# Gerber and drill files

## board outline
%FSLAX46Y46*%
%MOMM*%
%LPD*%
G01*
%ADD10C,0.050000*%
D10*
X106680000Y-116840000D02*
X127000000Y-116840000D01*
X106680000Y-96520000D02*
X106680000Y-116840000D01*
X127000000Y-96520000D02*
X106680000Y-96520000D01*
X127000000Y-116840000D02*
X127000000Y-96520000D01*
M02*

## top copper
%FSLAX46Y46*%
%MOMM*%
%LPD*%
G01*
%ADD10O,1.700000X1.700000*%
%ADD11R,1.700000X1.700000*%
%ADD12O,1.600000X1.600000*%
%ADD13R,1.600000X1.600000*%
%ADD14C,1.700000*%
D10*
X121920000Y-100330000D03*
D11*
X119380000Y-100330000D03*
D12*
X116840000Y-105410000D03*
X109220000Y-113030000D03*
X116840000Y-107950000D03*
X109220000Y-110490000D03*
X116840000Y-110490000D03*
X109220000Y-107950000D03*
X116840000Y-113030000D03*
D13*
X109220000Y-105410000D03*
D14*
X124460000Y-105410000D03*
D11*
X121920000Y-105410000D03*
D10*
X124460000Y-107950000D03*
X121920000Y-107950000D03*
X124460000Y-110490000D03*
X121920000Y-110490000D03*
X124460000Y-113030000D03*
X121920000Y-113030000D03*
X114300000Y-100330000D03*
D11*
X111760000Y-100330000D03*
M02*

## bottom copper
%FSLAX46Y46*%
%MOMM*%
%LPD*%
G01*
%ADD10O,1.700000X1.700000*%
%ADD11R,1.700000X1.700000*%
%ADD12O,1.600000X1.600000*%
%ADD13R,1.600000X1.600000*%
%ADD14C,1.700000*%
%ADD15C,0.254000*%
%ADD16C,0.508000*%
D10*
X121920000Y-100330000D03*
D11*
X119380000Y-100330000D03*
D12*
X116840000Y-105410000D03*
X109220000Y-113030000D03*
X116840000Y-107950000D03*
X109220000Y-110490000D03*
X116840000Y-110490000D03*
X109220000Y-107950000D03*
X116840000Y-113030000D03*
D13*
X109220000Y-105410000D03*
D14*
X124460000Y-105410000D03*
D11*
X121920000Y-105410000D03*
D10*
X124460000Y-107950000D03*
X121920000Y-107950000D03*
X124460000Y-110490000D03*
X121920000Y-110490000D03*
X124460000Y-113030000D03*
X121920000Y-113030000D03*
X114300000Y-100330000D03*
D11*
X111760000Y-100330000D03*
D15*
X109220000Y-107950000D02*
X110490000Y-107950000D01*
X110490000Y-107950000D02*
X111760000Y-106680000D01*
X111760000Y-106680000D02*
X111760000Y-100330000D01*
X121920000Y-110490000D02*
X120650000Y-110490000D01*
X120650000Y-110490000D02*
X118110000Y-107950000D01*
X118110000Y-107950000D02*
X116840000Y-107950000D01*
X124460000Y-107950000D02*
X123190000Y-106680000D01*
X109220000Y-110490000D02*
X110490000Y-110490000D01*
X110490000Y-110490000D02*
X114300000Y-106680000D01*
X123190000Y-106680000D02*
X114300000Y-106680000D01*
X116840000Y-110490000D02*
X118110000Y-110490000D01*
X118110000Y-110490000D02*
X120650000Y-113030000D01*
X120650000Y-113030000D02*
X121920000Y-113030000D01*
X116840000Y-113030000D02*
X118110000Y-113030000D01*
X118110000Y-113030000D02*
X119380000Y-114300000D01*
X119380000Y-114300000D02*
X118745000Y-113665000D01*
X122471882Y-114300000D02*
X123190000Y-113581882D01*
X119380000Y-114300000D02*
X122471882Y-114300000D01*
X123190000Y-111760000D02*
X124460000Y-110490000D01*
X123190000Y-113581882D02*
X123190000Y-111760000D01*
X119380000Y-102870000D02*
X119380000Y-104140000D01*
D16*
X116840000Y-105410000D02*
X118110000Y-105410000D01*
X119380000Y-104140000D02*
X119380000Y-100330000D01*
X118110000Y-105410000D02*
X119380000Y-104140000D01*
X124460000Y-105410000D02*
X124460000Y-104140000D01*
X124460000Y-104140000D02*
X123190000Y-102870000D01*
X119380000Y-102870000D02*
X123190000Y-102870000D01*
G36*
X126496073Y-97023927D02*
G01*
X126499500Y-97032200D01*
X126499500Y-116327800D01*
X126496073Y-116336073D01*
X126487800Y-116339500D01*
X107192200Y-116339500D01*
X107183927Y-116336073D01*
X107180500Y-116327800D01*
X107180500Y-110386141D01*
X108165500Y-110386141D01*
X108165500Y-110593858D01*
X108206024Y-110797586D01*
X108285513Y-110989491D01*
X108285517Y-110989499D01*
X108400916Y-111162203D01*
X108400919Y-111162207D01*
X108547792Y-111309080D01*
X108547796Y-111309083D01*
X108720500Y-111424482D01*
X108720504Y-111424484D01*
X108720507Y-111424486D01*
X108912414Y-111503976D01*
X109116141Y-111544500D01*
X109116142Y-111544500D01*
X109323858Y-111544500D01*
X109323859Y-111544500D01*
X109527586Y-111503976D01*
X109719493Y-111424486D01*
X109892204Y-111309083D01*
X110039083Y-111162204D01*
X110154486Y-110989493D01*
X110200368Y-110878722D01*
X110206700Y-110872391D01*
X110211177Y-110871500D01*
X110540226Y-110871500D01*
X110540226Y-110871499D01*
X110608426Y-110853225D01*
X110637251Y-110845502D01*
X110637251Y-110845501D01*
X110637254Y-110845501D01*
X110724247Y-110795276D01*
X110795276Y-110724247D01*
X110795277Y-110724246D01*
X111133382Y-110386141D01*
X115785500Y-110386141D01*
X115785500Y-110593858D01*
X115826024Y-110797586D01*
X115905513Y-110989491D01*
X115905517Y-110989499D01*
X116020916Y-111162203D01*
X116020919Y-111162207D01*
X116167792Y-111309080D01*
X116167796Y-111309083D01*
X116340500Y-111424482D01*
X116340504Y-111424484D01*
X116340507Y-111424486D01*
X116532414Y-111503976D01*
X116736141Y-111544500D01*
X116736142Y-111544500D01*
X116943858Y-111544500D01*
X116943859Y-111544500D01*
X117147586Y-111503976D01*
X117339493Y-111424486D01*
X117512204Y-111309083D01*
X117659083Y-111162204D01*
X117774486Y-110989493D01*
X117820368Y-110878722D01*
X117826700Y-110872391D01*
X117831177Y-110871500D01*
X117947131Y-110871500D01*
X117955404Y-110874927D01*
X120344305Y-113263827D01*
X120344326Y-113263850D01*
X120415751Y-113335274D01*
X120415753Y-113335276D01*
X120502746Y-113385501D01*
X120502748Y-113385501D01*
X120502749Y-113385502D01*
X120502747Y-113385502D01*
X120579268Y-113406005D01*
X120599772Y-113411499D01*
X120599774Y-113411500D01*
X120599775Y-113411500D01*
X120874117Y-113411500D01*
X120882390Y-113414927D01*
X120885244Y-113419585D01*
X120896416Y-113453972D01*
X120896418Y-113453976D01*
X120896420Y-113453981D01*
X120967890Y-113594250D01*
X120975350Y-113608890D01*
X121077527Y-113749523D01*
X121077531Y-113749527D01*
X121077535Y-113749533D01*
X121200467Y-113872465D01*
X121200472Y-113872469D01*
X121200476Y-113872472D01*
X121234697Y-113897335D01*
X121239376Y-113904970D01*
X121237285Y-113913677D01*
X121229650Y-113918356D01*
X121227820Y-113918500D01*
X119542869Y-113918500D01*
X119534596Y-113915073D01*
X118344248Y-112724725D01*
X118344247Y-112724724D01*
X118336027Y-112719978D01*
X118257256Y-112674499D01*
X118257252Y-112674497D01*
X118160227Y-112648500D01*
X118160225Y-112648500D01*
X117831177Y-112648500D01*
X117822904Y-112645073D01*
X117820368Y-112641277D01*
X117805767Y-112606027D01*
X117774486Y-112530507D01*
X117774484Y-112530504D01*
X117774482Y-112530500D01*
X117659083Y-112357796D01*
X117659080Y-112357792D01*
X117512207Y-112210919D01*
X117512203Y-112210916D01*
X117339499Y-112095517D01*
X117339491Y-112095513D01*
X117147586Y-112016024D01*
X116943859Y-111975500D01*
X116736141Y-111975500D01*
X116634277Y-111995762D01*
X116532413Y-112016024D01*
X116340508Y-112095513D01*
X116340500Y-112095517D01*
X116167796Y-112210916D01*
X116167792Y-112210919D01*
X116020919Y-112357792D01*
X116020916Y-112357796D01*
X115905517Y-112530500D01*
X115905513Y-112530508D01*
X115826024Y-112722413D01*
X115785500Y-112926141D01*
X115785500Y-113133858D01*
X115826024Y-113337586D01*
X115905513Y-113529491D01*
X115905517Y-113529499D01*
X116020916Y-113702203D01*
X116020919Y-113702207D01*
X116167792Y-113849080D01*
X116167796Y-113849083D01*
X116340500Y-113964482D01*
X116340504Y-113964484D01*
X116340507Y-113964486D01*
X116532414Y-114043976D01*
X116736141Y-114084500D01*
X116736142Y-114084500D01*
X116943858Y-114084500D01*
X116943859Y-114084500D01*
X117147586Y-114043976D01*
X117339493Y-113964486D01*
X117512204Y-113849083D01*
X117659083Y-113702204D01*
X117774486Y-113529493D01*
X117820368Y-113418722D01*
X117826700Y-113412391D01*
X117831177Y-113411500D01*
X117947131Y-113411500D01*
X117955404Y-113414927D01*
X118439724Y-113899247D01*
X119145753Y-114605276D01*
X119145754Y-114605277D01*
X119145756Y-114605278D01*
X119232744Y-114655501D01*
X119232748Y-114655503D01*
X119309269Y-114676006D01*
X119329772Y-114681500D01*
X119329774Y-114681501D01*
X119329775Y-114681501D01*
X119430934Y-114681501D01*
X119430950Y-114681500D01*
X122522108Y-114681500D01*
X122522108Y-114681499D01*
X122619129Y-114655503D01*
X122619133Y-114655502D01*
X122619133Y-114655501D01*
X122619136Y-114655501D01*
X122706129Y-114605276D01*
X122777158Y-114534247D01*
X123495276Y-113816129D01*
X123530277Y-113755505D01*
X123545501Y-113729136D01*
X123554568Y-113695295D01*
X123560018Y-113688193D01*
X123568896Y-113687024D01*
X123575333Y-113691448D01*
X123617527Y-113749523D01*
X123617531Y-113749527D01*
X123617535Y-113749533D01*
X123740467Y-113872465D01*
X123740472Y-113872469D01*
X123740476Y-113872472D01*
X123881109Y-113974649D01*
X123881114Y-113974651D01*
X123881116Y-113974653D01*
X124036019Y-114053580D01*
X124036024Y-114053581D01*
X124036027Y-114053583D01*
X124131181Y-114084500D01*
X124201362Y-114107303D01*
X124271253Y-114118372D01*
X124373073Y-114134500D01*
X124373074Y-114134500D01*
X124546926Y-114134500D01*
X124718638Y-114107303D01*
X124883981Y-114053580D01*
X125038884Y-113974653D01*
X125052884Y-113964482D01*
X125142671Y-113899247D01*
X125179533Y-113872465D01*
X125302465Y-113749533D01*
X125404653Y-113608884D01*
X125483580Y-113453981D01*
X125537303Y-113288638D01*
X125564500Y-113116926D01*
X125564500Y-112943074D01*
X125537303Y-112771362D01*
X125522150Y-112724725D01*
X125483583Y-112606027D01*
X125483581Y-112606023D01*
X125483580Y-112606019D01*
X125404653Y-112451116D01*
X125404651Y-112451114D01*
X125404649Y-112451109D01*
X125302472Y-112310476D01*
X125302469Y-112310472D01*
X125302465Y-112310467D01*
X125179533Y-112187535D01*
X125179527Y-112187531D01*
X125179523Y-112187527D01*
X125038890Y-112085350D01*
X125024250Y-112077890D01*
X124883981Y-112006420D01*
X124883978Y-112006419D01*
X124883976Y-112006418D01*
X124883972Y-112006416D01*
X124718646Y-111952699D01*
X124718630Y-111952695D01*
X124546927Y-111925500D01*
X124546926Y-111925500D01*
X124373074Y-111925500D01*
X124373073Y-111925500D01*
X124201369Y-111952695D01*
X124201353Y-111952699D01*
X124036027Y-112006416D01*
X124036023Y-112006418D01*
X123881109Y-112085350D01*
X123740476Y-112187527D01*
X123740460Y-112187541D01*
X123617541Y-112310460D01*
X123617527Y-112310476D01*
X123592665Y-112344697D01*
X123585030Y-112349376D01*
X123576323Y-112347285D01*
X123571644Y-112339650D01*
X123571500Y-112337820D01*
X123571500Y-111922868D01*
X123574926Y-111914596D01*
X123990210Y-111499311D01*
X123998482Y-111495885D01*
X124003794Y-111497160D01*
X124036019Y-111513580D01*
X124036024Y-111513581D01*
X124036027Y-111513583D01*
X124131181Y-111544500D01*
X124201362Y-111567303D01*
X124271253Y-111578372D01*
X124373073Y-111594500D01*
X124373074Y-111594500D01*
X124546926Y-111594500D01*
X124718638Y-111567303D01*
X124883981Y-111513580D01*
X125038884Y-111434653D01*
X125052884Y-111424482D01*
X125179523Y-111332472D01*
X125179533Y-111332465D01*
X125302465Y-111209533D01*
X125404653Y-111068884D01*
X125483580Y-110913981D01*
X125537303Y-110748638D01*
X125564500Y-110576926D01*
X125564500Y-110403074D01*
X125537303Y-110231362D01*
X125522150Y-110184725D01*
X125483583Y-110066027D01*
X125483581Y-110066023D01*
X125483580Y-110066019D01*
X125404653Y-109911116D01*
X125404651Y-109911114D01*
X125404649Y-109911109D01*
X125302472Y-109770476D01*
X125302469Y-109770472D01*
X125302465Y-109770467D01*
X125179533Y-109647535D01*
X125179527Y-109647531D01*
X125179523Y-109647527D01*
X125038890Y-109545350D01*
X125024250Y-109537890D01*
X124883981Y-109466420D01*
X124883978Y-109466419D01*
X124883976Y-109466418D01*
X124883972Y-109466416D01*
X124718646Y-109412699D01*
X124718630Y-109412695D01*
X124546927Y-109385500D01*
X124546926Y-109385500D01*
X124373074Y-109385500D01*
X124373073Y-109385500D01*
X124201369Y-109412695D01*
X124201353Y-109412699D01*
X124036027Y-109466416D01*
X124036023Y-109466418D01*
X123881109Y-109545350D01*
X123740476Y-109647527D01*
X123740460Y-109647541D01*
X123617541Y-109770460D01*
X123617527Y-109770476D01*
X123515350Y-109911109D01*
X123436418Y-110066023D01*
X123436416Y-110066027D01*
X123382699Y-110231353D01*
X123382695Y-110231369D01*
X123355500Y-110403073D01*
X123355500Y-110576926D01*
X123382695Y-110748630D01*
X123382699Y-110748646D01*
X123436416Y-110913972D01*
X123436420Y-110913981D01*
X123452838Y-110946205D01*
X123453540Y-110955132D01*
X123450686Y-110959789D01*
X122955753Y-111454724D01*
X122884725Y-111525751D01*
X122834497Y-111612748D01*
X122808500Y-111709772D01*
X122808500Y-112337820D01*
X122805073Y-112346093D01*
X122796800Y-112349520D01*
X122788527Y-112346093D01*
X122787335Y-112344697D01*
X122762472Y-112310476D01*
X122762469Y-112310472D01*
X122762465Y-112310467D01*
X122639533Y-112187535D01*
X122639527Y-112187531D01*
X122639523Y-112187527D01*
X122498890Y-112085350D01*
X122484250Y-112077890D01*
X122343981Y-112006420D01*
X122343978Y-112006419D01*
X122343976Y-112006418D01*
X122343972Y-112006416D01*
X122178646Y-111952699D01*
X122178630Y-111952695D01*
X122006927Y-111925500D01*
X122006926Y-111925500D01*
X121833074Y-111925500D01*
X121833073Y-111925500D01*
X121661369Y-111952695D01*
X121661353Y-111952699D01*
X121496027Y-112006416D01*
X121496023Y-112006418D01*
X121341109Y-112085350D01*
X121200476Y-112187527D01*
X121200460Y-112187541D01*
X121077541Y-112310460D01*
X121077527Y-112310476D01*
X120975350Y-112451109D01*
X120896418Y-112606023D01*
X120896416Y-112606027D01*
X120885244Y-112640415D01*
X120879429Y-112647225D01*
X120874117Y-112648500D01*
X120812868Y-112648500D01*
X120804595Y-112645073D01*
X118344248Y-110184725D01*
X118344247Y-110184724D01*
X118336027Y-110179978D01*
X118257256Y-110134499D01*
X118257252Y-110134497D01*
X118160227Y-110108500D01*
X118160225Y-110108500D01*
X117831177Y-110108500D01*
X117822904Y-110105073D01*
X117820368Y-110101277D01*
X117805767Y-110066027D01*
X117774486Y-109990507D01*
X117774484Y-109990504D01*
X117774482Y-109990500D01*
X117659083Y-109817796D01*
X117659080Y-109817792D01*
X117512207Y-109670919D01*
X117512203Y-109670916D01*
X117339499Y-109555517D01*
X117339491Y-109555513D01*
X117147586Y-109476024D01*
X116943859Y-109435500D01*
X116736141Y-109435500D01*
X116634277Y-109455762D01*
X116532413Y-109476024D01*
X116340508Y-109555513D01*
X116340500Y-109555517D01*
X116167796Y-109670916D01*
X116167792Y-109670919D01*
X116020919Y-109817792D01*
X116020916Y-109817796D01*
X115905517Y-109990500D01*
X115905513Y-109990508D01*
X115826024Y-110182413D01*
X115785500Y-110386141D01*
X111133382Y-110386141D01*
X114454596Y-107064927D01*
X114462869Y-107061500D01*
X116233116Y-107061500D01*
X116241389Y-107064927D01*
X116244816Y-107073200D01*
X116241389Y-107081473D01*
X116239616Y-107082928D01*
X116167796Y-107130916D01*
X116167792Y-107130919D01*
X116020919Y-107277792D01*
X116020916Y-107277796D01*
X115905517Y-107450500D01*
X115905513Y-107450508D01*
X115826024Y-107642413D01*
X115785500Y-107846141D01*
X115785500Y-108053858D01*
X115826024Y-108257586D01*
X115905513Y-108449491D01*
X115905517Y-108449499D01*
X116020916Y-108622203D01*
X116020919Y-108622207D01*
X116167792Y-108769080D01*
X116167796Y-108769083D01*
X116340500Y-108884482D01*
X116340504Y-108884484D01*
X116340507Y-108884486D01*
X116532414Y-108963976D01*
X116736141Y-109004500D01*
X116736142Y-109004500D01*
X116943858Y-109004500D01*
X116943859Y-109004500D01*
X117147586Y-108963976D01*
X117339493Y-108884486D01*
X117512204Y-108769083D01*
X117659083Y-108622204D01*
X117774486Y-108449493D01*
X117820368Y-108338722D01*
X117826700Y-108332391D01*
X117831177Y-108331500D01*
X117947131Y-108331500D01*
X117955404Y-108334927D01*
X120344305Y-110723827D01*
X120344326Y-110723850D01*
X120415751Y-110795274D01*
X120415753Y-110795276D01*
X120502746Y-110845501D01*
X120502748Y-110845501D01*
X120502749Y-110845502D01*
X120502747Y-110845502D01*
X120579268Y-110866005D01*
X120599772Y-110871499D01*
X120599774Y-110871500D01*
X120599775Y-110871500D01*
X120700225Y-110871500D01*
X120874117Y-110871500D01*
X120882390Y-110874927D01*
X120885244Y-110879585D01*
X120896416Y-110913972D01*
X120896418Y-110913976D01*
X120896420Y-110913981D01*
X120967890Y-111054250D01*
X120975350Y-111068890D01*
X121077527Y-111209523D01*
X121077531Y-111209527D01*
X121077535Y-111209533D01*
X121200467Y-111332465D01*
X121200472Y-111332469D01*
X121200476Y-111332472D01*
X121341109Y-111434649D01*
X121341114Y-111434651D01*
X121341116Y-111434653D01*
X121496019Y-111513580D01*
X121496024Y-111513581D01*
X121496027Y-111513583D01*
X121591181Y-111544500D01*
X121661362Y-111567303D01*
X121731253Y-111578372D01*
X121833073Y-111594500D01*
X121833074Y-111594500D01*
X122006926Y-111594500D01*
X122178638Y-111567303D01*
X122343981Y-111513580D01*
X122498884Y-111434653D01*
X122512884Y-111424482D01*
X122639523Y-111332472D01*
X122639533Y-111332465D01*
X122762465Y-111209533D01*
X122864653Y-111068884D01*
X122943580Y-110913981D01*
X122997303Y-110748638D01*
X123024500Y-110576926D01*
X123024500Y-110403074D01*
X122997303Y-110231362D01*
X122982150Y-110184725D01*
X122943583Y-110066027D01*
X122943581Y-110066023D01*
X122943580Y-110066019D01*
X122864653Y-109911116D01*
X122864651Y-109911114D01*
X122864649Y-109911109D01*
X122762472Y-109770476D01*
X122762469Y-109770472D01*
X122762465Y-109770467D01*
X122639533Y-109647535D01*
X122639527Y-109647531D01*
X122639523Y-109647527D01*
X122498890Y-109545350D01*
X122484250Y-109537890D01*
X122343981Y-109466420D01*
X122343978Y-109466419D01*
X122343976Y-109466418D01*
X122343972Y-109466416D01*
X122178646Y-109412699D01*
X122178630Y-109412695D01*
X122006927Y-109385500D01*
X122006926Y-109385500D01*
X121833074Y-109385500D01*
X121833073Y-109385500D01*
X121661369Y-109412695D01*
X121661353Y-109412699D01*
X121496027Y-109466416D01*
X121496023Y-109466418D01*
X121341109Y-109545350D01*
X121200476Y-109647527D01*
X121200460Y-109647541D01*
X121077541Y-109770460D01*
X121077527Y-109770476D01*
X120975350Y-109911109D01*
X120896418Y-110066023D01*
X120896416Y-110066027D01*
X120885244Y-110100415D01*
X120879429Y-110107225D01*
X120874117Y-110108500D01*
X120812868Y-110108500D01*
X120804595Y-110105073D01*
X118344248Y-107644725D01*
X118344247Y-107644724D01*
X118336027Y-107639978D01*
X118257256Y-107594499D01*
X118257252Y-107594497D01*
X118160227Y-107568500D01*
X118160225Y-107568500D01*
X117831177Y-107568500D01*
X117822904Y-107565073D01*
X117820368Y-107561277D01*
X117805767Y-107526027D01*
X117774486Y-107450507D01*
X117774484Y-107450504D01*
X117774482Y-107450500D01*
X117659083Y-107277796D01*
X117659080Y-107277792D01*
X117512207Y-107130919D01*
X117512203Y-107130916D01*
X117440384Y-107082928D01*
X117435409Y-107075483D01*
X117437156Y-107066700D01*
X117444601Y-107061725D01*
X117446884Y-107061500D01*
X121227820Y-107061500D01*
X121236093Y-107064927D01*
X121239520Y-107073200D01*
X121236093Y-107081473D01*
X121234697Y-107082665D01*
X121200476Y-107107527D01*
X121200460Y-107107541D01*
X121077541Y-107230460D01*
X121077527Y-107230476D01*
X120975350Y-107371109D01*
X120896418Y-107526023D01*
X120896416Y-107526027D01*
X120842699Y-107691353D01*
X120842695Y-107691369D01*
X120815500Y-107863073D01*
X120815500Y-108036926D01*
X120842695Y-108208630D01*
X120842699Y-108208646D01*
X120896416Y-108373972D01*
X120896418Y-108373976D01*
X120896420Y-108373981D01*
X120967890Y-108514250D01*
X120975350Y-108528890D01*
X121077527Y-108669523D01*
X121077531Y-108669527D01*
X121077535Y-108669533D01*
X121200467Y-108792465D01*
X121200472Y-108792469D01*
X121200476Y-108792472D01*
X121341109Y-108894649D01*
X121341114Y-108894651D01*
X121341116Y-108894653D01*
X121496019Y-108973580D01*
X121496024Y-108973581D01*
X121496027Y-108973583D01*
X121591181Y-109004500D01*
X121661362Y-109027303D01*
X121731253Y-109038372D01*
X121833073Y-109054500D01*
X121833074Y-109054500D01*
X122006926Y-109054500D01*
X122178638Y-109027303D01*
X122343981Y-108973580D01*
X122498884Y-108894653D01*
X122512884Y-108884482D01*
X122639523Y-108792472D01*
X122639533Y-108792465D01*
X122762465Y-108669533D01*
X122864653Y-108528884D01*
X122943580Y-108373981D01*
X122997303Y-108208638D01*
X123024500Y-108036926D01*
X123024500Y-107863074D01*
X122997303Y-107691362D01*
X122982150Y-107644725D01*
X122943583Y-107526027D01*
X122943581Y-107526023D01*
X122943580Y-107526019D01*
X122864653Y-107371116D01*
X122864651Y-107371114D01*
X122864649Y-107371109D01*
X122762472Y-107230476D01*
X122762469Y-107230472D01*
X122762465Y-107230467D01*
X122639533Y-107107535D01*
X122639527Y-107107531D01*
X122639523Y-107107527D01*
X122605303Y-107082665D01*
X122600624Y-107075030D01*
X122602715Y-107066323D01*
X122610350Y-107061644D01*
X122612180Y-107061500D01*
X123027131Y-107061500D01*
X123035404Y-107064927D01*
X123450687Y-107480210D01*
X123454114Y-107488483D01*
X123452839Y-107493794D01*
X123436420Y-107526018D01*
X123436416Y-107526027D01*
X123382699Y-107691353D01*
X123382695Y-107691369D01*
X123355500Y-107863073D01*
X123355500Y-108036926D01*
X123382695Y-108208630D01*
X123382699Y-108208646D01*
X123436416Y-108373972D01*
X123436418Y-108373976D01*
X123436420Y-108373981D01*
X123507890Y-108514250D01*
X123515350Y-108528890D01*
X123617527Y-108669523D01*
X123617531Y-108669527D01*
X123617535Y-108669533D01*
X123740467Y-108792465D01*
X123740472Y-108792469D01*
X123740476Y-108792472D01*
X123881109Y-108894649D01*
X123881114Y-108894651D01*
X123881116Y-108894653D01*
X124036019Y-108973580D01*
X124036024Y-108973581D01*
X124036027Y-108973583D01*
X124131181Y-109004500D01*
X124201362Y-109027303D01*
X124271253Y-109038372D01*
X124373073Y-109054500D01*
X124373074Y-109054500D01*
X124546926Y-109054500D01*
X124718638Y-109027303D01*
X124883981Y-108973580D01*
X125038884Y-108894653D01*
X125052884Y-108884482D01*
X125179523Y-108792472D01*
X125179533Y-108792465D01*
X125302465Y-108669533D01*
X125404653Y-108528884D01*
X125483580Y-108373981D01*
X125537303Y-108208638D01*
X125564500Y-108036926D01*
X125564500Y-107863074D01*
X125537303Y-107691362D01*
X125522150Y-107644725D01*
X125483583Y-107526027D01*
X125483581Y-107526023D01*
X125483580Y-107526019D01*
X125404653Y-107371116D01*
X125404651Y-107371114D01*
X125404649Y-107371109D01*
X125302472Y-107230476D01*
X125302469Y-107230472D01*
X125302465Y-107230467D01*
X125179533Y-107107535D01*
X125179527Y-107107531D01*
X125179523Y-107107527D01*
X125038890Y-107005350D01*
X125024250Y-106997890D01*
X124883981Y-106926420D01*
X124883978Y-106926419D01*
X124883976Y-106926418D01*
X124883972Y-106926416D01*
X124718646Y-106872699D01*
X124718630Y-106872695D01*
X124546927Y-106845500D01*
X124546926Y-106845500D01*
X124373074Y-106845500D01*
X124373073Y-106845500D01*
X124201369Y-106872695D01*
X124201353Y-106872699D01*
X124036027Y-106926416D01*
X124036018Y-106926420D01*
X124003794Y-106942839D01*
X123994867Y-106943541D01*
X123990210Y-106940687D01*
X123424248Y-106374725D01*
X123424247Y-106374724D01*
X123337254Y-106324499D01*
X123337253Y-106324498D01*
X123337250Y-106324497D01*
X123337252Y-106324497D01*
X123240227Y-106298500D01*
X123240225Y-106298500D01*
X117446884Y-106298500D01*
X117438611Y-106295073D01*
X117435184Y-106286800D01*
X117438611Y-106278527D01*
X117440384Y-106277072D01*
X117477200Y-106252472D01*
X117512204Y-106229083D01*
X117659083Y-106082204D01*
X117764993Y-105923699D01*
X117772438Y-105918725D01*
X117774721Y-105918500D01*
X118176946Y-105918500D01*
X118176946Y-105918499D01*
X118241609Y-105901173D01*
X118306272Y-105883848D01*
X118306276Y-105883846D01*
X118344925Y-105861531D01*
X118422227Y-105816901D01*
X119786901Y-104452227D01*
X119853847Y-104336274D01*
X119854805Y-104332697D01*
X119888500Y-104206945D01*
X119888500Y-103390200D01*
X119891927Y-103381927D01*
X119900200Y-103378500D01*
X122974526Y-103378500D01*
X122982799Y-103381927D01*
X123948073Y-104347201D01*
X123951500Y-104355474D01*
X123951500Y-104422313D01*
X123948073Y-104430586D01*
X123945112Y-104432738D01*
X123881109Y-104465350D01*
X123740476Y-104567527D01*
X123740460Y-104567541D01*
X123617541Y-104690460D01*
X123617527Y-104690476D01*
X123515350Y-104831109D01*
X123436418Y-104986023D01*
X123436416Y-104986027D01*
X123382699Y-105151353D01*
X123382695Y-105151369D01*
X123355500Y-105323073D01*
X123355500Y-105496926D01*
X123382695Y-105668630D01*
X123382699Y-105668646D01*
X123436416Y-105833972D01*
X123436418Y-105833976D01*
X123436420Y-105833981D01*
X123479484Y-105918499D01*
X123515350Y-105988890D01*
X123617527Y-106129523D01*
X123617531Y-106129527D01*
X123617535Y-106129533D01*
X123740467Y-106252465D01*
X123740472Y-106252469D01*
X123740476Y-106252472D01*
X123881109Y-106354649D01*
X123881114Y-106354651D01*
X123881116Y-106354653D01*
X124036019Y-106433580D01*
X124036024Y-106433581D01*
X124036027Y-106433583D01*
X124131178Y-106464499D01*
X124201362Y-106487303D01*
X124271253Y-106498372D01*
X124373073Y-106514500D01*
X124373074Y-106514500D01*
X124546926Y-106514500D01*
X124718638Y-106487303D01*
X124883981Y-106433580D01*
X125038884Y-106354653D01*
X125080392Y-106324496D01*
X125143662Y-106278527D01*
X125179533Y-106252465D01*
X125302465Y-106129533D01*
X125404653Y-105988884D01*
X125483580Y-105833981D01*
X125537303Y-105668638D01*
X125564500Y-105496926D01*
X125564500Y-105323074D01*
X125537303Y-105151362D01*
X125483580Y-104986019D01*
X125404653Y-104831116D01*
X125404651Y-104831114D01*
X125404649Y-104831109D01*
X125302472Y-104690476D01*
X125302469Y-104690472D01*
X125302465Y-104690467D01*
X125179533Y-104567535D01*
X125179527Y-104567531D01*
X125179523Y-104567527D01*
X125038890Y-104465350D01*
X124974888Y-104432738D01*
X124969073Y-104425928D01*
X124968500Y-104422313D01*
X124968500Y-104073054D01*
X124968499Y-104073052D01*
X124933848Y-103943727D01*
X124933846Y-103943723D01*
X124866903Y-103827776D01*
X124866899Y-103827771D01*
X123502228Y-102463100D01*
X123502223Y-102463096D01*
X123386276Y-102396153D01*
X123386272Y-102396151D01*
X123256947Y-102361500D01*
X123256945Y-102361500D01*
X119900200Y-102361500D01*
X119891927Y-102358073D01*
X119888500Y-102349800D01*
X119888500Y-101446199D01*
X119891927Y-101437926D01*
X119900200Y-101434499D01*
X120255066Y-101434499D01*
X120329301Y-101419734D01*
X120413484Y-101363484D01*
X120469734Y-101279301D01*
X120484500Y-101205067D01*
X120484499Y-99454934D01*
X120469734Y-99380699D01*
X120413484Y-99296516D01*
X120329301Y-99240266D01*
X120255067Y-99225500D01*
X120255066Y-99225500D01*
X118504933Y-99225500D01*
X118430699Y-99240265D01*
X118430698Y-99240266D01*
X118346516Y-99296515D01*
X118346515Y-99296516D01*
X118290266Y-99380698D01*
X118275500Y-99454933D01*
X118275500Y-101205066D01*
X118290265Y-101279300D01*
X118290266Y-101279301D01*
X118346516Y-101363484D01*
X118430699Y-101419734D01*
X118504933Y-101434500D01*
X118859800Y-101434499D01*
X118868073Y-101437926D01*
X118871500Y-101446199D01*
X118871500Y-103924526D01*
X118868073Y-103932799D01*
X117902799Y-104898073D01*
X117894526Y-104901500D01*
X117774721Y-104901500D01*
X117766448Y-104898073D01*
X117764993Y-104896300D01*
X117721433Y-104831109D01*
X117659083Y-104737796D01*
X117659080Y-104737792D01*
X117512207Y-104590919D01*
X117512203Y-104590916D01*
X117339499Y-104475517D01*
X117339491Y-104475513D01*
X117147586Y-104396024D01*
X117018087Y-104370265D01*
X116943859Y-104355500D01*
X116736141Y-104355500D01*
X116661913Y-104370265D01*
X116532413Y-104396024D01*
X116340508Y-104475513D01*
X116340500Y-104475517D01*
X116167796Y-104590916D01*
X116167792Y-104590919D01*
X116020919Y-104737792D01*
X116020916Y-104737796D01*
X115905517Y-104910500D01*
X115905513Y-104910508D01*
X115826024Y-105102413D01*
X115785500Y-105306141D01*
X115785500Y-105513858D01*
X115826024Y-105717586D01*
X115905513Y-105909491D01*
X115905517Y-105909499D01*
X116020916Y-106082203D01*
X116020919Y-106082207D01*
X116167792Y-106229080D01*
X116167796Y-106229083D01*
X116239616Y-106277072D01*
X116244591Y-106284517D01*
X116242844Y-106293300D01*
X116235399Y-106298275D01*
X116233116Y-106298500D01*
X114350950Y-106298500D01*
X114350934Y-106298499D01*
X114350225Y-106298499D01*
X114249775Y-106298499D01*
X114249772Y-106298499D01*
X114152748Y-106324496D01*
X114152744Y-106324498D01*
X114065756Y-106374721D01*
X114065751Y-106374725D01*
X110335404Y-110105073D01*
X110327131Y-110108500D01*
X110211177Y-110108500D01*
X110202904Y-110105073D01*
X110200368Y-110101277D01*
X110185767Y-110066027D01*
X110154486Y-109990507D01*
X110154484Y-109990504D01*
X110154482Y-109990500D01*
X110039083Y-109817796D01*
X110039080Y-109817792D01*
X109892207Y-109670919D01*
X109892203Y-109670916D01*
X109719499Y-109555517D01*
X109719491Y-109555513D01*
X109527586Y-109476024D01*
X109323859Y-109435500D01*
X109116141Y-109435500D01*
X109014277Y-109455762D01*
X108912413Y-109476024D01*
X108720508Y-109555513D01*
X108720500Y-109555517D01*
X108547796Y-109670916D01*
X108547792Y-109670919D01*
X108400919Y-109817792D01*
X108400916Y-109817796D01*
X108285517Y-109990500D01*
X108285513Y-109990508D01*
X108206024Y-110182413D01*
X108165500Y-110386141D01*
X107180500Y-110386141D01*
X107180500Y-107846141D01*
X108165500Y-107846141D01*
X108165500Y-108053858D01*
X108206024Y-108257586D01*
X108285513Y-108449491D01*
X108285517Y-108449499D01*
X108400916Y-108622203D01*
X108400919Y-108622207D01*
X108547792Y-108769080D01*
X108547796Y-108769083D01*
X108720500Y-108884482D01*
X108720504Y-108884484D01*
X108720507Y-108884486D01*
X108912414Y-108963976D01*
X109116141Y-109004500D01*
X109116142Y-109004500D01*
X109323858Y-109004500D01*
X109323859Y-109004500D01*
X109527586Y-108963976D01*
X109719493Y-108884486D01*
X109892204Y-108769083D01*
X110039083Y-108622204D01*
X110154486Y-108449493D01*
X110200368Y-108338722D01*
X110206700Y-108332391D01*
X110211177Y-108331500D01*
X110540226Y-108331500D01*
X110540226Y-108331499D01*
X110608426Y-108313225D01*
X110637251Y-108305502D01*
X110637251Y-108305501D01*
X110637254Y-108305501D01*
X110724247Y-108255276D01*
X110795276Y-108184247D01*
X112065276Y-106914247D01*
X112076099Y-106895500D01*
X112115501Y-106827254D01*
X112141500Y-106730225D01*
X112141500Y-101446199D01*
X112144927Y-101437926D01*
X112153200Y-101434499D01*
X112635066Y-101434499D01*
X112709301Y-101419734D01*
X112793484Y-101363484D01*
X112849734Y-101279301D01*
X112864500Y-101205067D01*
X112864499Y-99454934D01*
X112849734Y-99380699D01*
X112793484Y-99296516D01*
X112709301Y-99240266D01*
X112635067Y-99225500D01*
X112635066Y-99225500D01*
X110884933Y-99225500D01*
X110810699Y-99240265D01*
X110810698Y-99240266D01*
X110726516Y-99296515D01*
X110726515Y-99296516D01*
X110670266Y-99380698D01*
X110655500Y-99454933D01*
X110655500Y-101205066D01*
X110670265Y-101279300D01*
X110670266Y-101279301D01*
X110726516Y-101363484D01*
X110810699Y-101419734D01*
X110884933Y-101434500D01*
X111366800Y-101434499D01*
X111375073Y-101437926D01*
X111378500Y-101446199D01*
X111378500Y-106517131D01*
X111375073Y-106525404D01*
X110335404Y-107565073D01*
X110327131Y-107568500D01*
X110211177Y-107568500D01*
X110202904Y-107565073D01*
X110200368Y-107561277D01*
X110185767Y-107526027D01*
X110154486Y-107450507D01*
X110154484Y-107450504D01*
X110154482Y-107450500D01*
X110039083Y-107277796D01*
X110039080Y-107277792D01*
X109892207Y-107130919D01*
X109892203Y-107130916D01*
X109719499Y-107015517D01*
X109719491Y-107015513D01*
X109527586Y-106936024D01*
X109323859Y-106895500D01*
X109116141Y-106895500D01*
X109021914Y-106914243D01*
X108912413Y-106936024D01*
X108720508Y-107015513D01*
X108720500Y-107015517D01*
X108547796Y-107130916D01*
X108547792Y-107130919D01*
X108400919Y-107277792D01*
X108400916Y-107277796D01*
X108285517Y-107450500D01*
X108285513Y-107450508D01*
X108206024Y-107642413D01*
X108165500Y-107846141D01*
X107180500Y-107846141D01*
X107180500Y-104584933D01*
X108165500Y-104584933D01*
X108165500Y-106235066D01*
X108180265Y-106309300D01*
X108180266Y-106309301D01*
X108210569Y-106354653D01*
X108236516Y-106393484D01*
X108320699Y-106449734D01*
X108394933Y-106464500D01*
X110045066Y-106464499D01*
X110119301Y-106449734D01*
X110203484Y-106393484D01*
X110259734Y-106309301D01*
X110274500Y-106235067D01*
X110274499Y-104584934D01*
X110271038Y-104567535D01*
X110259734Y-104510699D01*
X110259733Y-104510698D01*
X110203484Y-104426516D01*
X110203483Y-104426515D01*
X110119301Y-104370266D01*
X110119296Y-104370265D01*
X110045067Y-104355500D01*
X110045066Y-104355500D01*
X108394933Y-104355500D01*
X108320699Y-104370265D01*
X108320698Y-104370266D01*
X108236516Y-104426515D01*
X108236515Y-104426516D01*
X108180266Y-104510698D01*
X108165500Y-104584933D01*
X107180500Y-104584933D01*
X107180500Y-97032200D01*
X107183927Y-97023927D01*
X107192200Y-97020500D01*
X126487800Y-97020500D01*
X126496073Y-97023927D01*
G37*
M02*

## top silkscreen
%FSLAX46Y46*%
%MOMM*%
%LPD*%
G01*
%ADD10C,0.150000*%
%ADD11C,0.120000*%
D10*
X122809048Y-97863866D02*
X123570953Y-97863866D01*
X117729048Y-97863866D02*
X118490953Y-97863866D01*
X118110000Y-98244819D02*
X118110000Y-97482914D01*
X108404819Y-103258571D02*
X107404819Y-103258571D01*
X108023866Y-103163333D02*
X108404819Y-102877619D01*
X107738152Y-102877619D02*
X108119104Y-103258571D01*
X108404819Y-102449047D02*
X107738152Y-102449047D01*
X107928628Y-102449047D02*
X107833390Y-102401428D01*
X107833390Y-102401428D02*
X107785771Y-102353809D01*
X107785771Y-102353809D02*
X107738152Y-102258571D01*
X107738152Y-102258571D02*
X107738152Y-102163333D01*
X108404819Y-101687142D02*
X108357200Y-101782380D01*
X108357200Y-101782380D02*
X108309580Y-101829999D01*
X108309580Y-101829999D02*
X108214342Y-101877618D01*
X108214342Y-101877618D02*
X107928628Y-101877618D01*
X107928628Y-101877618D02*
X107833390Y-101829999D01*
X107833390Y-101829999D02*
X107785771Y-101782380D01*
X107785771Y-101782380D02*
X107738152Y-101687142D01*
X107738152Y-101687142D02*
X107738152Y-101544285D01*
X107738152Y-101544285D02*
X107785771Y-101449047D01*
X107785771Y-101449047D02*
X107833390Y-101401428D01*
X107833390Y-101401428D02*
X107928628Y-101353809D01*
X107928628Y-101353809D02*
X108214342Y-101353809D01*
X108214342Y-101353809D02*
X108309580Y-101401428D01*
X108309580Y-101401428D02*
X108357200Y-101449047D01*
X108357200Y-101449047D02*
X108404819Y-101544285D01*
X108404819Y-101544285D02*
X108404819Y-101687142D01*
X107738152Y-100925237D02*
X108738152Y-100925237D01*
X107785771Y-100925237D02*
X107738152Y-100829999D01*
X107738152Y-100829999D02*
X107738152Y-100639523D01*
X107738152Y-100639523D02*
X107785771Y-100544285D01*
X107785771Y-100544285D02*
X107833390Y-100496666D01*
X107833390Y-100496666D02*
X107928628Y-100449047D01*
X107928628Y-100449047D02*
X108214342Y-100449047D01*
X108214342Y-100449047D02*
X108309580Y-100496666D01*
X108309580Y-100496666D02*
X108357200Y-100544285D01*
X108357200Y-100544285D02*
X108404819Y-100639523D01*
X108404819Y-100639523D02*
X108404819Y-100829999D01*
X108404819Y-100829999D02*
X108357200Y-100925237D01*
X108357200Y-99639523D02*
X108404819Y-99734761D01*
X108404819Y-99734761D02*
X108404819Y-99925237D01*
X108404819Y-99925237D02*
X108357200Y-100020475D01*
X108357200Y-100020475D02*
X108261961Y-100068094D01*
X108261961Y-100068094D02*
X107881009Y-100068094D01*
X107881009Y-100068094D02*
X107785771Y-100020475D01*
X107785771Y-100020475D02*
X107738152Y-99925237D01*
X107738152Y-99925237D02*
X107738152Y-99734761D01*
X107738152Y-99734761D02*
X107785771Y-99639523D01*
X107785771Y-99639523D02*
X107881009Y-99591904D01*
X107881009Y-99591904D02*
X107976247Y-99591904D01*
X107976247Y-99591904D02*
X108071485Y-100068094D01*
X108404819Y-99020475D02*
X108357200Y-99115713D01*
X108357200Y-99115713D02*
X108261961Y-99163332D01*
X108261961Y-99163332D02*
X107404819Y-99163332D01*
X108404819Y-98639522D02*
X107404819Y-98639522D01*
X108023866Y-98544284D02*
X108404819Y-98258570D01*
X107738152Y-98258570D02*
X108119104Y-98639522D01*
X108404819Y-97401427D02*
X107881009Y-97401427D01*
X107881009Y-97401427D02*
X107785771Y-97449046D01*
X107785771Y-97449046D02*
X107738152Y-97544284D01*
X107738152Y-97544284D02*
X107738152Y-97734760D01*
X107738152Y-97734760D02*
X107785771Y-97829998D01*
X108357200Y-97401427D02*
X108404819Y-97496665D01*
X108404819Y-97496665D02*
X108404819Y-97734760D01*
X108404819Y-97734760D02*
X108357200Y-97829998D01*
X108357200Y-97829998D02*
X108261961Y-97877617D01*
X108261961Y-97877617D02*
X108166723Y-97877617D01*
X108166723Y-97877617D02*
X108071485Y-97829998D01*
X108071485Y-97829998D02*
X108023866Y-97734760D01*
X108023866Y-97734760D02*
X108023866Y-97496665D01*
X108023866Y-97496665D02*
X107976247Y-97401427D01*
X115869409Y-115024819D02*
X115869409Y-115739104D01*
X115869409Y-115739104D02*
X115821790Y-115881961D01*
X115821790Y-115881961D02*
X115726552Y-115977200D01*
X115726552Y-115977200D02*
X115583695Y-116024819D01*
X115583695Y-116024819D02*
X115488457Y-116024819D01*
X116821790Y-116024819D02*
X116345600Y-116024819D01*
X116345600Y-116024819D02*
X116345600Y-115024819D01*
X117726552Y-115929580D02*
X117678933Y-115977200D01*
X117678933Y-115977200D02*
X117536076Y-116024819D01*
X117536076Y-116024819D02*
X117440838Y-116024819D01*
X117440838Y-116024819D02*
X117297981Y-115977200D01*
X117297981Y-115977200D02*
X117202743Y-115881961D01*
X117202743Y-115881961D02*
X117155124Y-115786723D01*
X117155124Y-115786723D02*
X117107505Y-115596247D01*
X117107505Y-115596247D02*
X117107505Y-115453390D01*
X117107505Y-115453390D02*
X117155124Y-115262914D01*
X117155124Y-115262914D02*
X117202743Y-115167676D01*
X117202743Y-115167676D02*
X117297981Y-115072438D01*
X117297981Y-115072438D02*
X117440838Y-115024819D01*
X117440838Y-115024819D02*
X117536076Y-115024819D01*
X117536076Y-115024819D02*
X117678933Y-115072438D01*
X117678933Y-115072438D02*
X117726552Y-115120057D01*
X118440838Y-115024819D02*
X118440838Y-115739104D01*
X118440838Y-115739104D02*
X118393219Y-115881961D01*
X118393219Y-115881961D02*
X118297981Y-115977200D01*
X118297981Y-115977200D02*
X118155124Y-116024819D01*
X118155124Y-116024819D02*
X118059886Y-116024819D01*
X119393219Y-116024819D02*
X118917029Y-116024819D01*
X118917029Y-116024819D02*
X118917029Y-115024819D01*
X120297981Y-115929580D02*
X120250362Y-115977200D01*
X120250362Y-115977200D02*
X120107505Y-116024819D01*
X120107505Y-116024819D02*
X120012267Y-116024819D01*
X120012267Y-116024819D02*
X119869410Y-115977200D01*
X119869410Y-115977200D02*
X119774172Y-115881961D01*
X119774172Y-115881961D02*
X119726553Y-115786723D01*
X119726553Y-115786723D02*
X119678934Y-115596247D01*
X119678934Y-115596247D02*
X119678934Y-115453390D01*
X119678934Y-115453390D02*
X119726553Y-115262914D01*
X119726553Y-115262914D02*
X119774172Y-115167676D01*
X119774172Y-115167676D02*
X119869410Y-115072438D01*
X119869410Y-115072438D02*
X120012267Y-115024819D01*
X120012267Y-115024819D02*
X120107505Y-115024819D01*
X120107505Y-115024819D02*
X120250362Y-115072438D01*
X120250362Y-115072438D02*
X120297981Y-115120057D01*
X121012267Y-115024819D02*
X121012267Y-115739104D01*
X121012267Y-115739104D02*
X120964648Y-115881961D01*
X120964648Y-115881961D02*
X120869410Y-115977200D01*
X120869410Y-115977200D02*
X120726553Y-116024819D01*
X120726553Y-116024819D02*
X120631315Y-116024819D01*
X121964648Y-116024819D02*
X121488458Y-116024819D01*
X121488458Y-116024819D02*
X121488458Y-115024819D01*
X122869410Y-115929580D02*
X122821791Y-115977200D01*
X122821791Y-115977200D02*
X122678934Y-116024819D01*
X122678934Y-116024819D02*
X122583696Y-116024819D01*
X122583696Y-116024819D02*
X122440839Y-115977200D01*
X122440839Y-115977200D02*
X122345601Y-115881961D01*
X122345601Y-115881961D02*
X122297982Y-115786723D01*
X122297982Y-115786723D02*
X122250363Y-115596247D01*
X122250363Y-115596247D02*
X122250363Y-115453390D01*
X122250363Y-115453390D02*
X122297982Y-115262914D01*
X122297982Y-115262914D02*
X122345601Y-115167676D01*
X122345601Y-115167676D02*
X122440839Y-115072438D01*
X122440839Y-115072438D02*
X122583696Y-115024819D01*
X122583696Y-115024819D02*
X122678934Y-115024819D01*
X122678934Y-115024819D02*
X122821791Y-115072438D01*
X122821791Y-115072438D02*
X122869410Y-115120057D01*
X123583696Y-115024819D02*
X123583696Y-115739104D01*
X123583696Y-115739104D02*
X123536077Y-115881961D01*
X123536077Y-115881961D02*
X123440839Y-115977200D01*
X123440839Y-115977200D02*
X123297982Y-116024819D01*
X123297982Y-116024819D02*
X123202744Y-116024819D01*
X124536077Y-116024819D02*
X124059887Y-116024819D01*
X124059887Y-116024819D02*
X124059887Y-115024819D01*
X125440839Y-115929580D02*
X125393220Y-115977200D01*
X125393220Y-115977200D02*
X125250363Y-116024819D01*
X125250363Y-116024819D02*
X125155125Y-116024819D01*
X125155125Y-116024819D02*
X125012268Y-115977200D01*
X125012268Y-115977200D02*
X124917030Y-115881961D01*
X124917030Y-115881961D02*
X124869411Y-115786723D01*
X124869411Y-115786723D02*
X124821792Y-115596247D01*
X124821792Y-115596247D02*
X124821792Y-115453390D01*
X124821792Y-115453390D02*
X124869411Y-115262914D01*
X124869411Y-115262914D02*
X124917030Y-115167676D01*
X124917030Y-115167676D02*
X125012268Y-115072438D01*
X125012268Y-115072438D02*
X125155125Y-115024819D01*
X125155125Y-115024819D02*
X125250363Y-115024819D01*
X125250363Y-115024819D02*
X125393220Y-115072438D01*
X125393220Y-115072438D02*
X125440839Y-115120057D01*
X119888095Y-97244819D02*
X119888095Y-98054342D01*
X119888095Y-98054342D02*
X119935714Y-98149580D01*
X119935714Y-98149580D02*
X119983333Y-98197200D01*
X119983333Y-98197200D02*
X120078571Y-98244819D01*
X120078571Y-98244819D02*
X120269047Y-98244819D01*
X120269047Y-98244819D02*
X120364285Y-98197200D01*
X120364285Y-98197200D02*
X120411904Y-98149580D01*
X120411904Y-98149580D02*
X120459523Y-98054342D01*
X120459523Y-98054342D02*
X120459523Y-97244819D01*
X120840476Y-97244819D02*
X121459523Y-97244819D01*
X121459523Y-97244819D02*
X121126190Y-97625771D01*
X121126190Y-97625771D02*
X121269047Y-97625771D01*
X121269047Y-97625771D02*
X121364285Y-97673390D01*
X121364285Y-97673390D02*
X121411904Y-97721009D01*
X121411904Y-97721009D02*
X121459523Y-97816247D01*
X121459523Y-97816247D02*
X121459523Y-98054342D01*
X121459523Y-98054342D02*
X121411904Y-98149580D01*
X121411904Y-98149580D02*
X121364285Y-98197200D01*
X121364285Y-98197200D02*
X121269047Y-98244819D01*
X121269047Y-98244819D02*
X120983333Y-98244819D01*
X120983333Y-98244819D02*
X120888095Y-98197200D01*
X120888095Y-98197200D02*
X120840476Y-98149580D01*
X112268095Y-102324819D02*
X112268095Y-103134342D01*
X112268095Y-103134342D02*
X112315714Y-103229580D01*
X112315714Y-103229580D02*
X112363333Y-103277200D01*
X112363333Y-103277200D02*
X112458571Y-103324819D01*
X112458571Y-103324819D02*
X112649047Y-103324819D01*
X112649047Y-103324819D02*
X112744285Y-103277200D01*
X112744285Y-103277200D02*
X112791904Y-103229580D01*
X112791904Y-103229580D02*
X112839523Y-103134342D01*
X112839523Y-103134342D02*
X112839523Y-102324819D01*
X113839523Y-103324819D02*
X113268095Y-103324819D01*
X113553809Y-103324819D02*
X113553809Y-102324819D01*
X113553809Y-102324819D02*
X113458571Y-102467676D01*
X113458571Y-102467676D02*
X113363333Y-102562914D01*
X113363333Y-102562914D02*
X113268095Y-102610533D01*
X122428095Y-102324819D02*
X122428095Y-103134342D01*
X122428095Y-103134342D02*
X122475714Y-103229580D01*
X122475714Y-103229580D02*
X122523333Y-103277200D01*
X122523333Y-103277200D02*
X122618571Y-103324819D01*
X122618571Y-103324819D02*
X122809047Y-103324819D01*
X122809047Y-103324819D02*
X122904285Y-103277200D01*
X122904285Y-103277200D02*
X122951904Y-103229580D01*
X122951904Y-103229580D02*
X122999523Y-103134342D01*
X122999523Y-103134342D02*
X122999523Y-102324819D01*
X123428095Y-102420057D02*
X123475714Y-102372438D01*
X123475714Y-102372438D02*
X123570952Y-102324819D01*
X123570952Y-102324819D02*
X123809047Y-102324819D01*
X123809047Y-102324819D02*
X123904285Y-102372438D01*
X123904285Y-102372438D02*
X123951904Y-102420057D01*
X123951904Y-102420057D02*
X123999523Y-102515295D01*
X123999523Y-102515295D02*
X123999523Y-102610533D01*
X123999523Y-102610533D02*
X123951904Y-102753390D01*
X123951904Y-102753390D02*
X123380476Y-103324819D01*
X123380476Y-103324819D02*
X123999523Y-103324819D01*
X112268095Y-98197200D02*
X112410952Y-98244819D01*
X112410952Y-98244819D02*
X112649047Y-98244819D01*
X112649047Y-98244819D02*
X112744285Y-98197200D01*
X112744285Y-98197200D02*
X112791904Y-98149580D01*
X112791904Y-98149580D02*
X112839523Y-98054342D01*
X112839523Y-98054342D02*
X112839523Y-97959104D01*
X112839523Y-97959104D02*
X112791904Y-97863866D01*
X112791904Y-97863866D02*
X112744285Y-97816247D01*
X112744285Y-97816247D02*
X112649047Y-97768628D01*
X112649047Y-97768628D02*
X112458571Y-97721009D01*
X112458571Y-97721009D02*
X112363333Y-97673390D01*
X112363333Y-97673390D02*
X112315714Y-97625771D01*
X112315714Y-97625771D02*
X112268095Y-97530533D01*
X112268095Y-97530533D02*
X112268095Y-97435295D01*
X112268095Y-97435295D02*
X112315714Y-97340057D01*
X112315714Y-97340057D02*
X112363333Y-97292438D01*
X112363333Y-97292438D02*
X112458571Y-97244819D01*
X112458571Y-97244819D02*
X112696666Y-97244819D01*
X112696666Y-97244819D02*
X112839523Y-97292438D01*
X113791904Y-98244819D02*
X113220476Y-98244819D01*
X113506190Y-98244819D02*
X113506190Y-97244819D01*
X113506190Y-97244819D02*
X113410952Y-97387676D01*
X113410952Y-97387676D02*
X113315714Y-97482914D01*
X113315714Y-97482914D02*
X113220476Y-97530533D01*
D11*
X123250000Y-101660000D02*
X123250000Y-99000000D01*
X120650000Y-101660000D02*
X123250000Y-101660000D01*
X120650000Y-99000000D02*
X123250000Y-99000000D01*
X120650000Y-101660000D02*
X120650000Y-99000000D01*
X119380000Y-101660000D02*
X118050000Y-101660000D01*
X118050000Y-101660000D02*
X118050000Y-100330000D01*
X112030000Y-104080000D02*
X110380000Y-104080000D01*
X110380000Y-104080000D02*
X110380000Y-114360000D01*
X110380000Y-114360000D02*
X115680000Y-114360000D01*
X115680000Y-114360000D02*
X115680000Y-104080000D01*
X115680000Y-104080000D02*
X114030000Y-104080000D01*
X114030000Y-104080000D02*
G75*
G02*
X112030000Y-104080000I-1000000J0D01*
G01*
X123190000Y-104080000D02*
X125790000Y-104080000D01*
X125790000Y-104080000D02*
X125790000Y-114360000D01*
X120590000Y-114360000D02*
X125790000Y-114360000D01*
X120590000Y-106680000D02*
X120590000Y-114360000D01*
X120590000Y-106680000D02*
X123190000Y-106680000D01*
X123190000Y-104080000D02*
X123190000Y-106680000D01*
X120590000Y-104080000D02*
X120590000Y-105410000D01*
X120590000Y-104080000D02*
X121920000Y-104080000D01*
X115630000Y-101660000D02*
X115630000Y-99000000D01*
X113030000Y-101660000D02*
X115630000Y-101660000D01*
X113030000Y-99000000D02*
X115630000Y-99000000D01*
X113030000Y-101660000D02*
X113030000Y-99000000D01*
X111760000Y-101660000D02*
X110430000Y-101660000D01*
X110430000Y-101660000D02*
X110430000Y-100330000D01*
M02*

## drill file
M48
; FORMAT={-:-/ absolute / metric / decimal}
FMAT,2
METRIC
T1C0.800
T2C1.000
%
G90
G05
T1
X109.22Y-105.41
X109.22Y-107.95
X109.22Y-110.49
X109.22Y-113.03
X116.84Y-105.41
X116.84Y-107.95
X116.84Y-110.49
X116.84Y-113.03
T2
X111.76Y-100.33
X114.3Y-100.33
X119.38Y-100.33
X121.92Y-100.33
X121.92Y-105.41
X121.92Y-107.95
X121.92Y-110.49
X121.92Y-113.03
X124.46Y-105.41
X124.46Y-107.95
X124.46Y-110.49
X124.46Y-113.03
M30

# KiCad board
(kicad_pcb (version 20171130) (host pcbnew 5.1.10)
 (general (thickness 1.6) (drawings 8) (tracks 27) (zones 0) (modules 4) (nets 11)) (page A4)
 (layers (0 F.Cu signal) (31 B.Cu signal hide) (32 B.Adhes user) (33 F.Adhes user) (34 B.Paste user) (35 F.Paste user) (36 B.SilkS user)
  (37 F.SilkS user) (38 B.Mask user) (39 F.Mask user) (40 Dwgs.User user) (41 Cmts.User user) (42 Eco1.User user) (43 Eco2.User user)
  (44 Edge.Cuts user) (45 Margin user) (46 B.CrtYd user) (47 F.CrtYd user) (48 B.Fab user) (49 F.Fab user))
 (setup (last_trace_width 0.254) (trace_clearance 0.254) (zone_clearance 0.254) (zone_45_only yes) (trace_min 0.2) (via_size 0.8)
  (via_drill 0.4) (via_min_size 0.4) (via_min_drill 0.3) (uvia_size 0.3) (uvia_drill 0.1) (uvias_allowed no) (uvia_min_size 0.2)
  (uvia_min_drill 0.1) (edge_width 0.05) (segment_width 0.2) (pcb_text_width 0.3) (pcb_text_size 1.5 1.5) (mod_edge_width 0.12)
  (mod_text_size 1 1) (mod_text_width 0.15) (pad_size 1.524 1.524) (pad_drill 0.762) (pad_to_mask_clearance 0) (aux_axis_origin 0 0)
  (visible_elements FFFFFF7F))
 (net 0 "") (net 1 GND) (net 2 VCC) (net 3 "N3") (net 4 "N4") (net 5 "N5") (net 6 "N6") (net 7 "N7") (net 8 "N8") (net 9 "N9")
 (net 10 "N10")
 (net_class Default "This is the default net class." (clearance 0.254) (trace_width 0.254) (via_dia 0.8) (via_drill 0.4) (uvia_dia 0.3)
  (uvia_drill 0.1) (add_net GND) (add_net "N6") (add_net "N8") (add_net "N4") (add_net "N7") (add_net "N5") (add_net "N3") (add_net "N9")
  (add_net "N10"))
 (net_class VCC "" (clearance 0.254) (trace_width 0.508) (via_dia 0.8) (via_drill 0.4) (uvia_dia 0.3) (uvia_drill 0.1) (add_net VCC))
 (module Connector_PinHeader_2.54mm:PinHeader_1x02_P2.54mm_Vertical (layer F.Cu) (at 119.38 100.33 90)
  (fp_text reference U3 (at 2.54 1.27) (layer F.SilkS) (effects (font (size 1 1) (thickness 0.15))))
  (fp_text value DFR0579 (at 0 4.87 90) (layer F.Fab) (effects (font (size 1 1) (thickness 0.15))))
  (fp_line (start -1.33 3.87) (end 1.33 3.87) (layer F.SilkS) (width 0.12))
  (fp_line (start -1.33 1.27) (end -1.33 3.87) (layer F.SilkS) (width 0.12))
  (fp_line (start 1.33 1.27) (end 1.33 3.87) (layer F.SilkS) (width 0.12))
  (fp_line (start -1.33 1.27) (end 1.33 1.27) (layer F.SilkS) (width 0.12))
  (fp_line (start -1.33 0) (end -1.33 -1.33) (layer F.SilkS) (width 0.12))
  (fp_line (start -1.33 -1.33) (end 0 -1.33) (layer F.SilkS) (width 0.12))
  (pad 2 thru_hole oval (at 0 2.54 90) (size 1.7 1.7) (drill 1) (layers *.Cu *.Mask) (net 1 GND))
  (pad 1 thru_hole rect (at 0 0 90) (size 1.7 1.7) (drill 1) (layers *.Cu *.Mask) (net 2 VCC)))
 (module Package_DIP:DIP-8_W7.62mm (layer F.Cu) (at 109.22 105.41)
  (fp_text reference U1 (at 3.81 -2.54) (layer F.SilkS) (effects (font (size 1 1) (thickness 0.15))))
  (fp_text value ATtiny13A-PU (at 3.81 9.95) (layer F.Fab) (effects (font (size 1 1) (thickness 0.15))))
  (fp_line (start 2.81 -1.33) (end 1.16 -1.33) (layer F.SilkS) (width 0.12))
  (fp_line (start 1.16 -1.33) (end 1.16 8.95) (layer F.SilkS) (width 0.12))
  (fp_line (start 1.16 8.95) (end 6.46 8.95) (layer F.SilkS) (width 0.12))
  (fp_line (start 6.46 8.95) (end 6.46 -1.33) (layer F.SilkS) (width 0.12))
  (fp_line (start 6.46 -1.33) (end 4.81 -1.33) (layer F.SilkS) (width 0.12))
  (fp_arc (start 3.81 -1.33) (end 2.81 -1.33) (angle -180) (layer F.SilkS) (width 0.12))
  (pad 8 thru_hole oval (at 7.62 0) (size 1.6 1.6) (drill 0.8) (layers *.Cu *.Mask) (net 2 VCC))
  (pad 4 thru_hole oval (at 0 7.62) (size 1.6 1.6) (drill 0.8) (layers *.Cu *.Mask) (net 1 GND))
  (pad 7 thru_hole oval (at 7.62 2.54) (size 1.6 1.6) (drill 0.8) (layers *.Cu *.Mask) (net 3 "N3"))
  (pad 3 thru_hole oval (at 0 5.08) (size 1.6 1.6) (drill 0.8) (layers *.Cu *.Mask) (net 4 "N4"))
  (pad 6 thru_hole oval (at 7.62 5.08) (size 1.6 1.6) (drill 0.8) (layers *.Cu *.Mask) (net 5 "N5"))
  (pad 2 thru_hole oval (at 0 2.54) (size 1.6 1.6) (drill 0.8) (layers *.Cu *.Mask) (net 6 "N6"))
  (pad 5 thru_hole oval (at 7.62 7.62) (size 1.6 1.6) (drill 0.8) (layers *.Cu *.Mask) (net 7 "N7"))
  (pad 1 thru_hole rect (at 0 0) (size 1.6 1.6) (drill 0.8) (layers *.Cu *.Mask) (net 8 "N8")))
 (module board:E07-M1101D (layer F.Cu) (at 121.92 105.41)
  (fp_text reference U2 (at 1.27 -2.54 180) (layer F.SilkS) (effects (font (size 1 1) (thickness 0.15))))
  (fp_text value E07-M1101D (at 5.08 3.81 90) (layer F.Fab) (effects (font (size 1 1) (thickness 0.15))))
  (fp_line (start 1.27 -1.33) (end 3.87 -1.33) (layer F.SilkS) (width 0.12))
  (fp_line (start 3.87 -1.33) (end 3.87 8.95) (layer F.SilkS) (width 0.12))
  (fp_line (start -1.33 8.95) (end 3.87 8.95) (layer F.SilkS) (width 0.12))
  (fp_line (start -1.33 1.27) (end -1.33 8.95) (layer F.SilkS) (width 0.12))
  (fp_line (start -1.33 1.27) (end 1.27 1.27) (layer F.SilkS) (width 0.12))
  (fp_line (start 1.27 -1.33) (end 1.27 1.27) (layer F.SilkS) (width 0.12))
  (fp_line (start -1.33 -1.33) (end -1.33 0) (layer F.SilkS) (width 0.12))
  (fp_line (start -1.33 -1.33) (end 0 -1.33) (layer F.SilkS) (width 0.12))
  (pad 2 thru_hole circle (at 2.54 0) (size 1.7 1.7) (drill 1) (layers *.Cu *.Mask) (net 2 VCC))
  (pad 1 thru_hole rect (at 0 0) (size 1.7 1.7) (drill 1) (layers *.Cu *.Mask) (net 1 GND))
  (pad 4 thru_hole oval (at 2.54 2.54) (size 1.7 1.7) (drill 1) (layers *.Cu *.Mask) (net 4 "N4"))
  (pad 3 thru_hole oval (at 0 2.54) (size 1.7 1.7) (drill 1) (layers *.Cu *.Mask) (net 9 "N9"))
  (pad 6 thru_hole oval (at 2.54 5.08) (size 1.7 1.7) (drill 1) (layers *.Cu *.Mask) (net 7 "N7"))
  (pad 5 thru_hole oval (at 0 5.08) (size 1.7 1.7) (drill 1) (layers *.Cu *.Mask) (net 3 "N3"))
  (pad 8 thru_hole oval (at 2.54 7.62) (size 1.7 1.7) (drill 1) (layers *.Cu *.Mask) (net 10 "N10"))
  (pad 7 thru_hole oval (at 0 7.62) (size 1.7 1.7) (drill 1) (layers *.Cu *.Mask) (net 5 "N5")))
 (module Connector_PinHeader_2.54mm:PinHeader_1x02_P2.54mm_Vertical (layer F.Cu) (at 111.76 100.33 90)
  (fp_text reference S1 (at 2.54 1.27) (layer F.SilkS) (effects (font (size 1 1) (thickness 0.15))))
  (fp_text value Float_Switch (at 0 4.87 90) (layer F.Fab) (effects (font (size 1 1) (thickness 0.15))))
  (fp_line (start -1.33 3.87) (end 1.33 3.87) (layer F.SilkS) (width 0.12))
  (fp_line (start -1.33 1.27) (end -1.33 3.87) (layer F.SilkS) (width 0.12))
  (fp_line (start 1.33 1.27) (end 1.33 3.87) (layer F.SilkS) (width 0.12))
  (fp_line (start -1.33 1.27) (end 1.33 1.27) (layer F.SilkS) (width 0.12))
  (fp_line (start -1.33 0) (end -1.33 -1.33) (layer F.SilkS) (width 0.12))
  (fp_line (start -1.33 -1.33) (end 0 -1.33) (layer F.SilkS) (width 0.12))
  (pad 2 thru_hole oval (at 0 2.54 90) (size 1.7 1.7) (drill 1) (layers *.Cu *.Mask) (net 1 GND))
  (pad 1 thru_hole rect (at 0 0 90) (size 1.7 1.7) (drill 1) (layers *.Cu *.Mask) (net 6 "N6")))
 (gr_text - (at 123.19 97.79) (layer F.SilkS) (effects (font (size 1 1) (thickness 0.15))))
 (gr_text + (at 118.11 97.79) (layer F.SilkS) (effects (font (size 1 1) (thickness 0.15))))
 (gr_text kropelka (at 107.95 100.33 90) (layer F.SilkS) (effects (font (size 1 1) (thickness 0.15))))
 (gr_line (start 106.68 116.84) (end 127 116.84) (layer Edge.Cuts) (width 0.05))
 (gr_line (start 106.68 96.52) (end 106.68 116.84) (layer Edge.Cuts) (width 0.05))
 (gr_line (start 127 96.52) (end 106.68 96.52) (layer Edge.Cuts) (width 0.05))
 (gr_line (start 127 116.84) (end 127 96.52) (layer Edge.Cuts) (width 0.05))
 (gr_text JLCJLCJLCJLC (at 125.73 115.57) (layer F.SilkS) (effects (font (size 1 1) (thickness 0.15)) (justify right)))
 (segment (start 109.22 107.95) (end 110.49 107.95) (width 0.254) (layer B.Cu) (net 6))
 (segment (start 110.49 107.95) (end 111.76 106.68) (width 0.254) (layer B.Cu) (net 6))
 (segment (start 111.76 106.68) (end 111.76 100.33) (width 0.254) (layer B.Cu) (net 6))
 (segment (start 121.92 110.49) (end 120.65 110.49) (width 0.254) (layer B.Cu) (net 3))
 (segment (start 120.65 110.49) (end 118.11 107.95) (width 0.254) (layer B.Cu) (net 3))
 (segment (start 118.11 107.95) (end 116.84 107.95) (width 0.254) (layer B.Cu) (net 3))
 (segment (start 124.46 107.95) (end 123.19 106.68) (width 0.254) (layer B.Cu) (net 4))
 (segment (start 109.22 110.49) (end 110.49 110.49) (width 0.254) (layer B.Cu) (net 4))
 (segment (start 110.49 110.49) (end 114.3 106.68) (width 0.254) (layer B.Cu) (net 4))
 (segment (start 123.19 106.68) (end 114.3 106.68) (width 0.254) (layer B.Cu) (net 4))
 (segment (start 116.84 110.49) (end 118.11 110.49) (width 0.254) (layer B.Cu) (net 5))
 (segment (start 118.11 110.49) (end 120.65 113.03) (width 0.254) (layer B.Cu) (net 5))
 (segment (start 120.65 113.03) (end 121.92 113.03) (width 0.254) (layer B.Cu) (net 5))
 (segment (start 116.84 113.03) (end 118.11 113.03) (width 0.254) (layer B.Cu) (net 7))
 (segment (start 118.11 113.03) (end 119.38 114.3) (width 0.254) (layer B.Cu) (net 7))
 (segment (start 119.38 114.3) (end 118.745 113.665) (width 0.254) (layer B.Cu) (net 7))
 (segment (start 122.471882 114.3) (end 123.19 113.581882) (width 0.254) (layer B.Cu) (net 7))
 (segment (start 119.38 114.3) (end 122.471882 114.3) (width 0.254) (layer B.Cu) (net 7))
 (segment (start 123.19 111.76) (end 124.46 110.49) (width 0.254) (layer B.Cu) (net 7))
 (segment (start 123.19 113.581882) (end 123.19 111.76) (width 0.254) (layer B.Cu) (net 7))
 (segment (start 119.38 102.87) (end 119.38 104.14) (width 0.254) (layer B.Cu) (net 2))
 (segment (start 116.84 105.41) (end 118.11 105.41) (width 0.508) (layer B.Cu) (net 2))
 (segment (start 119.38 104.14) (end 119.38 100.33) (width 0.508) (layer B.Cu) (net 2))
 (segment (start 118.11 105.41) (end 119.38 104.14) (width 0.508) (layer B.Cu) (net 2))
 (segment (start 124.46 105.41) (end 124.46 104.14) (width 0.508) (layer B.Cu) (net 2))
 (segment (start 124.46 104.14) (end 123.19 102.87) (width 0.508) (layer B.Cu) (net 2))
 (segment (start 119.38 102.87) (end 123.19 102.87) (width 0.508) (layer B.Cu) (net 2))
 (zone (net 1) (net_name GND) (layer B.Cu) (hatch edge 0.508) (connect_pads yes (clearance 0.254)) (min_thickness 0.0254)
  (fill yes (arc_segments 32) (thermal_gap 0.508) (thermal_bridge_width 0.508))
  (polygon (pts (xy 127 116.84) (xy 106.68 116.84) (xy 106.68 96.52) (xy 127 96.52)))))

